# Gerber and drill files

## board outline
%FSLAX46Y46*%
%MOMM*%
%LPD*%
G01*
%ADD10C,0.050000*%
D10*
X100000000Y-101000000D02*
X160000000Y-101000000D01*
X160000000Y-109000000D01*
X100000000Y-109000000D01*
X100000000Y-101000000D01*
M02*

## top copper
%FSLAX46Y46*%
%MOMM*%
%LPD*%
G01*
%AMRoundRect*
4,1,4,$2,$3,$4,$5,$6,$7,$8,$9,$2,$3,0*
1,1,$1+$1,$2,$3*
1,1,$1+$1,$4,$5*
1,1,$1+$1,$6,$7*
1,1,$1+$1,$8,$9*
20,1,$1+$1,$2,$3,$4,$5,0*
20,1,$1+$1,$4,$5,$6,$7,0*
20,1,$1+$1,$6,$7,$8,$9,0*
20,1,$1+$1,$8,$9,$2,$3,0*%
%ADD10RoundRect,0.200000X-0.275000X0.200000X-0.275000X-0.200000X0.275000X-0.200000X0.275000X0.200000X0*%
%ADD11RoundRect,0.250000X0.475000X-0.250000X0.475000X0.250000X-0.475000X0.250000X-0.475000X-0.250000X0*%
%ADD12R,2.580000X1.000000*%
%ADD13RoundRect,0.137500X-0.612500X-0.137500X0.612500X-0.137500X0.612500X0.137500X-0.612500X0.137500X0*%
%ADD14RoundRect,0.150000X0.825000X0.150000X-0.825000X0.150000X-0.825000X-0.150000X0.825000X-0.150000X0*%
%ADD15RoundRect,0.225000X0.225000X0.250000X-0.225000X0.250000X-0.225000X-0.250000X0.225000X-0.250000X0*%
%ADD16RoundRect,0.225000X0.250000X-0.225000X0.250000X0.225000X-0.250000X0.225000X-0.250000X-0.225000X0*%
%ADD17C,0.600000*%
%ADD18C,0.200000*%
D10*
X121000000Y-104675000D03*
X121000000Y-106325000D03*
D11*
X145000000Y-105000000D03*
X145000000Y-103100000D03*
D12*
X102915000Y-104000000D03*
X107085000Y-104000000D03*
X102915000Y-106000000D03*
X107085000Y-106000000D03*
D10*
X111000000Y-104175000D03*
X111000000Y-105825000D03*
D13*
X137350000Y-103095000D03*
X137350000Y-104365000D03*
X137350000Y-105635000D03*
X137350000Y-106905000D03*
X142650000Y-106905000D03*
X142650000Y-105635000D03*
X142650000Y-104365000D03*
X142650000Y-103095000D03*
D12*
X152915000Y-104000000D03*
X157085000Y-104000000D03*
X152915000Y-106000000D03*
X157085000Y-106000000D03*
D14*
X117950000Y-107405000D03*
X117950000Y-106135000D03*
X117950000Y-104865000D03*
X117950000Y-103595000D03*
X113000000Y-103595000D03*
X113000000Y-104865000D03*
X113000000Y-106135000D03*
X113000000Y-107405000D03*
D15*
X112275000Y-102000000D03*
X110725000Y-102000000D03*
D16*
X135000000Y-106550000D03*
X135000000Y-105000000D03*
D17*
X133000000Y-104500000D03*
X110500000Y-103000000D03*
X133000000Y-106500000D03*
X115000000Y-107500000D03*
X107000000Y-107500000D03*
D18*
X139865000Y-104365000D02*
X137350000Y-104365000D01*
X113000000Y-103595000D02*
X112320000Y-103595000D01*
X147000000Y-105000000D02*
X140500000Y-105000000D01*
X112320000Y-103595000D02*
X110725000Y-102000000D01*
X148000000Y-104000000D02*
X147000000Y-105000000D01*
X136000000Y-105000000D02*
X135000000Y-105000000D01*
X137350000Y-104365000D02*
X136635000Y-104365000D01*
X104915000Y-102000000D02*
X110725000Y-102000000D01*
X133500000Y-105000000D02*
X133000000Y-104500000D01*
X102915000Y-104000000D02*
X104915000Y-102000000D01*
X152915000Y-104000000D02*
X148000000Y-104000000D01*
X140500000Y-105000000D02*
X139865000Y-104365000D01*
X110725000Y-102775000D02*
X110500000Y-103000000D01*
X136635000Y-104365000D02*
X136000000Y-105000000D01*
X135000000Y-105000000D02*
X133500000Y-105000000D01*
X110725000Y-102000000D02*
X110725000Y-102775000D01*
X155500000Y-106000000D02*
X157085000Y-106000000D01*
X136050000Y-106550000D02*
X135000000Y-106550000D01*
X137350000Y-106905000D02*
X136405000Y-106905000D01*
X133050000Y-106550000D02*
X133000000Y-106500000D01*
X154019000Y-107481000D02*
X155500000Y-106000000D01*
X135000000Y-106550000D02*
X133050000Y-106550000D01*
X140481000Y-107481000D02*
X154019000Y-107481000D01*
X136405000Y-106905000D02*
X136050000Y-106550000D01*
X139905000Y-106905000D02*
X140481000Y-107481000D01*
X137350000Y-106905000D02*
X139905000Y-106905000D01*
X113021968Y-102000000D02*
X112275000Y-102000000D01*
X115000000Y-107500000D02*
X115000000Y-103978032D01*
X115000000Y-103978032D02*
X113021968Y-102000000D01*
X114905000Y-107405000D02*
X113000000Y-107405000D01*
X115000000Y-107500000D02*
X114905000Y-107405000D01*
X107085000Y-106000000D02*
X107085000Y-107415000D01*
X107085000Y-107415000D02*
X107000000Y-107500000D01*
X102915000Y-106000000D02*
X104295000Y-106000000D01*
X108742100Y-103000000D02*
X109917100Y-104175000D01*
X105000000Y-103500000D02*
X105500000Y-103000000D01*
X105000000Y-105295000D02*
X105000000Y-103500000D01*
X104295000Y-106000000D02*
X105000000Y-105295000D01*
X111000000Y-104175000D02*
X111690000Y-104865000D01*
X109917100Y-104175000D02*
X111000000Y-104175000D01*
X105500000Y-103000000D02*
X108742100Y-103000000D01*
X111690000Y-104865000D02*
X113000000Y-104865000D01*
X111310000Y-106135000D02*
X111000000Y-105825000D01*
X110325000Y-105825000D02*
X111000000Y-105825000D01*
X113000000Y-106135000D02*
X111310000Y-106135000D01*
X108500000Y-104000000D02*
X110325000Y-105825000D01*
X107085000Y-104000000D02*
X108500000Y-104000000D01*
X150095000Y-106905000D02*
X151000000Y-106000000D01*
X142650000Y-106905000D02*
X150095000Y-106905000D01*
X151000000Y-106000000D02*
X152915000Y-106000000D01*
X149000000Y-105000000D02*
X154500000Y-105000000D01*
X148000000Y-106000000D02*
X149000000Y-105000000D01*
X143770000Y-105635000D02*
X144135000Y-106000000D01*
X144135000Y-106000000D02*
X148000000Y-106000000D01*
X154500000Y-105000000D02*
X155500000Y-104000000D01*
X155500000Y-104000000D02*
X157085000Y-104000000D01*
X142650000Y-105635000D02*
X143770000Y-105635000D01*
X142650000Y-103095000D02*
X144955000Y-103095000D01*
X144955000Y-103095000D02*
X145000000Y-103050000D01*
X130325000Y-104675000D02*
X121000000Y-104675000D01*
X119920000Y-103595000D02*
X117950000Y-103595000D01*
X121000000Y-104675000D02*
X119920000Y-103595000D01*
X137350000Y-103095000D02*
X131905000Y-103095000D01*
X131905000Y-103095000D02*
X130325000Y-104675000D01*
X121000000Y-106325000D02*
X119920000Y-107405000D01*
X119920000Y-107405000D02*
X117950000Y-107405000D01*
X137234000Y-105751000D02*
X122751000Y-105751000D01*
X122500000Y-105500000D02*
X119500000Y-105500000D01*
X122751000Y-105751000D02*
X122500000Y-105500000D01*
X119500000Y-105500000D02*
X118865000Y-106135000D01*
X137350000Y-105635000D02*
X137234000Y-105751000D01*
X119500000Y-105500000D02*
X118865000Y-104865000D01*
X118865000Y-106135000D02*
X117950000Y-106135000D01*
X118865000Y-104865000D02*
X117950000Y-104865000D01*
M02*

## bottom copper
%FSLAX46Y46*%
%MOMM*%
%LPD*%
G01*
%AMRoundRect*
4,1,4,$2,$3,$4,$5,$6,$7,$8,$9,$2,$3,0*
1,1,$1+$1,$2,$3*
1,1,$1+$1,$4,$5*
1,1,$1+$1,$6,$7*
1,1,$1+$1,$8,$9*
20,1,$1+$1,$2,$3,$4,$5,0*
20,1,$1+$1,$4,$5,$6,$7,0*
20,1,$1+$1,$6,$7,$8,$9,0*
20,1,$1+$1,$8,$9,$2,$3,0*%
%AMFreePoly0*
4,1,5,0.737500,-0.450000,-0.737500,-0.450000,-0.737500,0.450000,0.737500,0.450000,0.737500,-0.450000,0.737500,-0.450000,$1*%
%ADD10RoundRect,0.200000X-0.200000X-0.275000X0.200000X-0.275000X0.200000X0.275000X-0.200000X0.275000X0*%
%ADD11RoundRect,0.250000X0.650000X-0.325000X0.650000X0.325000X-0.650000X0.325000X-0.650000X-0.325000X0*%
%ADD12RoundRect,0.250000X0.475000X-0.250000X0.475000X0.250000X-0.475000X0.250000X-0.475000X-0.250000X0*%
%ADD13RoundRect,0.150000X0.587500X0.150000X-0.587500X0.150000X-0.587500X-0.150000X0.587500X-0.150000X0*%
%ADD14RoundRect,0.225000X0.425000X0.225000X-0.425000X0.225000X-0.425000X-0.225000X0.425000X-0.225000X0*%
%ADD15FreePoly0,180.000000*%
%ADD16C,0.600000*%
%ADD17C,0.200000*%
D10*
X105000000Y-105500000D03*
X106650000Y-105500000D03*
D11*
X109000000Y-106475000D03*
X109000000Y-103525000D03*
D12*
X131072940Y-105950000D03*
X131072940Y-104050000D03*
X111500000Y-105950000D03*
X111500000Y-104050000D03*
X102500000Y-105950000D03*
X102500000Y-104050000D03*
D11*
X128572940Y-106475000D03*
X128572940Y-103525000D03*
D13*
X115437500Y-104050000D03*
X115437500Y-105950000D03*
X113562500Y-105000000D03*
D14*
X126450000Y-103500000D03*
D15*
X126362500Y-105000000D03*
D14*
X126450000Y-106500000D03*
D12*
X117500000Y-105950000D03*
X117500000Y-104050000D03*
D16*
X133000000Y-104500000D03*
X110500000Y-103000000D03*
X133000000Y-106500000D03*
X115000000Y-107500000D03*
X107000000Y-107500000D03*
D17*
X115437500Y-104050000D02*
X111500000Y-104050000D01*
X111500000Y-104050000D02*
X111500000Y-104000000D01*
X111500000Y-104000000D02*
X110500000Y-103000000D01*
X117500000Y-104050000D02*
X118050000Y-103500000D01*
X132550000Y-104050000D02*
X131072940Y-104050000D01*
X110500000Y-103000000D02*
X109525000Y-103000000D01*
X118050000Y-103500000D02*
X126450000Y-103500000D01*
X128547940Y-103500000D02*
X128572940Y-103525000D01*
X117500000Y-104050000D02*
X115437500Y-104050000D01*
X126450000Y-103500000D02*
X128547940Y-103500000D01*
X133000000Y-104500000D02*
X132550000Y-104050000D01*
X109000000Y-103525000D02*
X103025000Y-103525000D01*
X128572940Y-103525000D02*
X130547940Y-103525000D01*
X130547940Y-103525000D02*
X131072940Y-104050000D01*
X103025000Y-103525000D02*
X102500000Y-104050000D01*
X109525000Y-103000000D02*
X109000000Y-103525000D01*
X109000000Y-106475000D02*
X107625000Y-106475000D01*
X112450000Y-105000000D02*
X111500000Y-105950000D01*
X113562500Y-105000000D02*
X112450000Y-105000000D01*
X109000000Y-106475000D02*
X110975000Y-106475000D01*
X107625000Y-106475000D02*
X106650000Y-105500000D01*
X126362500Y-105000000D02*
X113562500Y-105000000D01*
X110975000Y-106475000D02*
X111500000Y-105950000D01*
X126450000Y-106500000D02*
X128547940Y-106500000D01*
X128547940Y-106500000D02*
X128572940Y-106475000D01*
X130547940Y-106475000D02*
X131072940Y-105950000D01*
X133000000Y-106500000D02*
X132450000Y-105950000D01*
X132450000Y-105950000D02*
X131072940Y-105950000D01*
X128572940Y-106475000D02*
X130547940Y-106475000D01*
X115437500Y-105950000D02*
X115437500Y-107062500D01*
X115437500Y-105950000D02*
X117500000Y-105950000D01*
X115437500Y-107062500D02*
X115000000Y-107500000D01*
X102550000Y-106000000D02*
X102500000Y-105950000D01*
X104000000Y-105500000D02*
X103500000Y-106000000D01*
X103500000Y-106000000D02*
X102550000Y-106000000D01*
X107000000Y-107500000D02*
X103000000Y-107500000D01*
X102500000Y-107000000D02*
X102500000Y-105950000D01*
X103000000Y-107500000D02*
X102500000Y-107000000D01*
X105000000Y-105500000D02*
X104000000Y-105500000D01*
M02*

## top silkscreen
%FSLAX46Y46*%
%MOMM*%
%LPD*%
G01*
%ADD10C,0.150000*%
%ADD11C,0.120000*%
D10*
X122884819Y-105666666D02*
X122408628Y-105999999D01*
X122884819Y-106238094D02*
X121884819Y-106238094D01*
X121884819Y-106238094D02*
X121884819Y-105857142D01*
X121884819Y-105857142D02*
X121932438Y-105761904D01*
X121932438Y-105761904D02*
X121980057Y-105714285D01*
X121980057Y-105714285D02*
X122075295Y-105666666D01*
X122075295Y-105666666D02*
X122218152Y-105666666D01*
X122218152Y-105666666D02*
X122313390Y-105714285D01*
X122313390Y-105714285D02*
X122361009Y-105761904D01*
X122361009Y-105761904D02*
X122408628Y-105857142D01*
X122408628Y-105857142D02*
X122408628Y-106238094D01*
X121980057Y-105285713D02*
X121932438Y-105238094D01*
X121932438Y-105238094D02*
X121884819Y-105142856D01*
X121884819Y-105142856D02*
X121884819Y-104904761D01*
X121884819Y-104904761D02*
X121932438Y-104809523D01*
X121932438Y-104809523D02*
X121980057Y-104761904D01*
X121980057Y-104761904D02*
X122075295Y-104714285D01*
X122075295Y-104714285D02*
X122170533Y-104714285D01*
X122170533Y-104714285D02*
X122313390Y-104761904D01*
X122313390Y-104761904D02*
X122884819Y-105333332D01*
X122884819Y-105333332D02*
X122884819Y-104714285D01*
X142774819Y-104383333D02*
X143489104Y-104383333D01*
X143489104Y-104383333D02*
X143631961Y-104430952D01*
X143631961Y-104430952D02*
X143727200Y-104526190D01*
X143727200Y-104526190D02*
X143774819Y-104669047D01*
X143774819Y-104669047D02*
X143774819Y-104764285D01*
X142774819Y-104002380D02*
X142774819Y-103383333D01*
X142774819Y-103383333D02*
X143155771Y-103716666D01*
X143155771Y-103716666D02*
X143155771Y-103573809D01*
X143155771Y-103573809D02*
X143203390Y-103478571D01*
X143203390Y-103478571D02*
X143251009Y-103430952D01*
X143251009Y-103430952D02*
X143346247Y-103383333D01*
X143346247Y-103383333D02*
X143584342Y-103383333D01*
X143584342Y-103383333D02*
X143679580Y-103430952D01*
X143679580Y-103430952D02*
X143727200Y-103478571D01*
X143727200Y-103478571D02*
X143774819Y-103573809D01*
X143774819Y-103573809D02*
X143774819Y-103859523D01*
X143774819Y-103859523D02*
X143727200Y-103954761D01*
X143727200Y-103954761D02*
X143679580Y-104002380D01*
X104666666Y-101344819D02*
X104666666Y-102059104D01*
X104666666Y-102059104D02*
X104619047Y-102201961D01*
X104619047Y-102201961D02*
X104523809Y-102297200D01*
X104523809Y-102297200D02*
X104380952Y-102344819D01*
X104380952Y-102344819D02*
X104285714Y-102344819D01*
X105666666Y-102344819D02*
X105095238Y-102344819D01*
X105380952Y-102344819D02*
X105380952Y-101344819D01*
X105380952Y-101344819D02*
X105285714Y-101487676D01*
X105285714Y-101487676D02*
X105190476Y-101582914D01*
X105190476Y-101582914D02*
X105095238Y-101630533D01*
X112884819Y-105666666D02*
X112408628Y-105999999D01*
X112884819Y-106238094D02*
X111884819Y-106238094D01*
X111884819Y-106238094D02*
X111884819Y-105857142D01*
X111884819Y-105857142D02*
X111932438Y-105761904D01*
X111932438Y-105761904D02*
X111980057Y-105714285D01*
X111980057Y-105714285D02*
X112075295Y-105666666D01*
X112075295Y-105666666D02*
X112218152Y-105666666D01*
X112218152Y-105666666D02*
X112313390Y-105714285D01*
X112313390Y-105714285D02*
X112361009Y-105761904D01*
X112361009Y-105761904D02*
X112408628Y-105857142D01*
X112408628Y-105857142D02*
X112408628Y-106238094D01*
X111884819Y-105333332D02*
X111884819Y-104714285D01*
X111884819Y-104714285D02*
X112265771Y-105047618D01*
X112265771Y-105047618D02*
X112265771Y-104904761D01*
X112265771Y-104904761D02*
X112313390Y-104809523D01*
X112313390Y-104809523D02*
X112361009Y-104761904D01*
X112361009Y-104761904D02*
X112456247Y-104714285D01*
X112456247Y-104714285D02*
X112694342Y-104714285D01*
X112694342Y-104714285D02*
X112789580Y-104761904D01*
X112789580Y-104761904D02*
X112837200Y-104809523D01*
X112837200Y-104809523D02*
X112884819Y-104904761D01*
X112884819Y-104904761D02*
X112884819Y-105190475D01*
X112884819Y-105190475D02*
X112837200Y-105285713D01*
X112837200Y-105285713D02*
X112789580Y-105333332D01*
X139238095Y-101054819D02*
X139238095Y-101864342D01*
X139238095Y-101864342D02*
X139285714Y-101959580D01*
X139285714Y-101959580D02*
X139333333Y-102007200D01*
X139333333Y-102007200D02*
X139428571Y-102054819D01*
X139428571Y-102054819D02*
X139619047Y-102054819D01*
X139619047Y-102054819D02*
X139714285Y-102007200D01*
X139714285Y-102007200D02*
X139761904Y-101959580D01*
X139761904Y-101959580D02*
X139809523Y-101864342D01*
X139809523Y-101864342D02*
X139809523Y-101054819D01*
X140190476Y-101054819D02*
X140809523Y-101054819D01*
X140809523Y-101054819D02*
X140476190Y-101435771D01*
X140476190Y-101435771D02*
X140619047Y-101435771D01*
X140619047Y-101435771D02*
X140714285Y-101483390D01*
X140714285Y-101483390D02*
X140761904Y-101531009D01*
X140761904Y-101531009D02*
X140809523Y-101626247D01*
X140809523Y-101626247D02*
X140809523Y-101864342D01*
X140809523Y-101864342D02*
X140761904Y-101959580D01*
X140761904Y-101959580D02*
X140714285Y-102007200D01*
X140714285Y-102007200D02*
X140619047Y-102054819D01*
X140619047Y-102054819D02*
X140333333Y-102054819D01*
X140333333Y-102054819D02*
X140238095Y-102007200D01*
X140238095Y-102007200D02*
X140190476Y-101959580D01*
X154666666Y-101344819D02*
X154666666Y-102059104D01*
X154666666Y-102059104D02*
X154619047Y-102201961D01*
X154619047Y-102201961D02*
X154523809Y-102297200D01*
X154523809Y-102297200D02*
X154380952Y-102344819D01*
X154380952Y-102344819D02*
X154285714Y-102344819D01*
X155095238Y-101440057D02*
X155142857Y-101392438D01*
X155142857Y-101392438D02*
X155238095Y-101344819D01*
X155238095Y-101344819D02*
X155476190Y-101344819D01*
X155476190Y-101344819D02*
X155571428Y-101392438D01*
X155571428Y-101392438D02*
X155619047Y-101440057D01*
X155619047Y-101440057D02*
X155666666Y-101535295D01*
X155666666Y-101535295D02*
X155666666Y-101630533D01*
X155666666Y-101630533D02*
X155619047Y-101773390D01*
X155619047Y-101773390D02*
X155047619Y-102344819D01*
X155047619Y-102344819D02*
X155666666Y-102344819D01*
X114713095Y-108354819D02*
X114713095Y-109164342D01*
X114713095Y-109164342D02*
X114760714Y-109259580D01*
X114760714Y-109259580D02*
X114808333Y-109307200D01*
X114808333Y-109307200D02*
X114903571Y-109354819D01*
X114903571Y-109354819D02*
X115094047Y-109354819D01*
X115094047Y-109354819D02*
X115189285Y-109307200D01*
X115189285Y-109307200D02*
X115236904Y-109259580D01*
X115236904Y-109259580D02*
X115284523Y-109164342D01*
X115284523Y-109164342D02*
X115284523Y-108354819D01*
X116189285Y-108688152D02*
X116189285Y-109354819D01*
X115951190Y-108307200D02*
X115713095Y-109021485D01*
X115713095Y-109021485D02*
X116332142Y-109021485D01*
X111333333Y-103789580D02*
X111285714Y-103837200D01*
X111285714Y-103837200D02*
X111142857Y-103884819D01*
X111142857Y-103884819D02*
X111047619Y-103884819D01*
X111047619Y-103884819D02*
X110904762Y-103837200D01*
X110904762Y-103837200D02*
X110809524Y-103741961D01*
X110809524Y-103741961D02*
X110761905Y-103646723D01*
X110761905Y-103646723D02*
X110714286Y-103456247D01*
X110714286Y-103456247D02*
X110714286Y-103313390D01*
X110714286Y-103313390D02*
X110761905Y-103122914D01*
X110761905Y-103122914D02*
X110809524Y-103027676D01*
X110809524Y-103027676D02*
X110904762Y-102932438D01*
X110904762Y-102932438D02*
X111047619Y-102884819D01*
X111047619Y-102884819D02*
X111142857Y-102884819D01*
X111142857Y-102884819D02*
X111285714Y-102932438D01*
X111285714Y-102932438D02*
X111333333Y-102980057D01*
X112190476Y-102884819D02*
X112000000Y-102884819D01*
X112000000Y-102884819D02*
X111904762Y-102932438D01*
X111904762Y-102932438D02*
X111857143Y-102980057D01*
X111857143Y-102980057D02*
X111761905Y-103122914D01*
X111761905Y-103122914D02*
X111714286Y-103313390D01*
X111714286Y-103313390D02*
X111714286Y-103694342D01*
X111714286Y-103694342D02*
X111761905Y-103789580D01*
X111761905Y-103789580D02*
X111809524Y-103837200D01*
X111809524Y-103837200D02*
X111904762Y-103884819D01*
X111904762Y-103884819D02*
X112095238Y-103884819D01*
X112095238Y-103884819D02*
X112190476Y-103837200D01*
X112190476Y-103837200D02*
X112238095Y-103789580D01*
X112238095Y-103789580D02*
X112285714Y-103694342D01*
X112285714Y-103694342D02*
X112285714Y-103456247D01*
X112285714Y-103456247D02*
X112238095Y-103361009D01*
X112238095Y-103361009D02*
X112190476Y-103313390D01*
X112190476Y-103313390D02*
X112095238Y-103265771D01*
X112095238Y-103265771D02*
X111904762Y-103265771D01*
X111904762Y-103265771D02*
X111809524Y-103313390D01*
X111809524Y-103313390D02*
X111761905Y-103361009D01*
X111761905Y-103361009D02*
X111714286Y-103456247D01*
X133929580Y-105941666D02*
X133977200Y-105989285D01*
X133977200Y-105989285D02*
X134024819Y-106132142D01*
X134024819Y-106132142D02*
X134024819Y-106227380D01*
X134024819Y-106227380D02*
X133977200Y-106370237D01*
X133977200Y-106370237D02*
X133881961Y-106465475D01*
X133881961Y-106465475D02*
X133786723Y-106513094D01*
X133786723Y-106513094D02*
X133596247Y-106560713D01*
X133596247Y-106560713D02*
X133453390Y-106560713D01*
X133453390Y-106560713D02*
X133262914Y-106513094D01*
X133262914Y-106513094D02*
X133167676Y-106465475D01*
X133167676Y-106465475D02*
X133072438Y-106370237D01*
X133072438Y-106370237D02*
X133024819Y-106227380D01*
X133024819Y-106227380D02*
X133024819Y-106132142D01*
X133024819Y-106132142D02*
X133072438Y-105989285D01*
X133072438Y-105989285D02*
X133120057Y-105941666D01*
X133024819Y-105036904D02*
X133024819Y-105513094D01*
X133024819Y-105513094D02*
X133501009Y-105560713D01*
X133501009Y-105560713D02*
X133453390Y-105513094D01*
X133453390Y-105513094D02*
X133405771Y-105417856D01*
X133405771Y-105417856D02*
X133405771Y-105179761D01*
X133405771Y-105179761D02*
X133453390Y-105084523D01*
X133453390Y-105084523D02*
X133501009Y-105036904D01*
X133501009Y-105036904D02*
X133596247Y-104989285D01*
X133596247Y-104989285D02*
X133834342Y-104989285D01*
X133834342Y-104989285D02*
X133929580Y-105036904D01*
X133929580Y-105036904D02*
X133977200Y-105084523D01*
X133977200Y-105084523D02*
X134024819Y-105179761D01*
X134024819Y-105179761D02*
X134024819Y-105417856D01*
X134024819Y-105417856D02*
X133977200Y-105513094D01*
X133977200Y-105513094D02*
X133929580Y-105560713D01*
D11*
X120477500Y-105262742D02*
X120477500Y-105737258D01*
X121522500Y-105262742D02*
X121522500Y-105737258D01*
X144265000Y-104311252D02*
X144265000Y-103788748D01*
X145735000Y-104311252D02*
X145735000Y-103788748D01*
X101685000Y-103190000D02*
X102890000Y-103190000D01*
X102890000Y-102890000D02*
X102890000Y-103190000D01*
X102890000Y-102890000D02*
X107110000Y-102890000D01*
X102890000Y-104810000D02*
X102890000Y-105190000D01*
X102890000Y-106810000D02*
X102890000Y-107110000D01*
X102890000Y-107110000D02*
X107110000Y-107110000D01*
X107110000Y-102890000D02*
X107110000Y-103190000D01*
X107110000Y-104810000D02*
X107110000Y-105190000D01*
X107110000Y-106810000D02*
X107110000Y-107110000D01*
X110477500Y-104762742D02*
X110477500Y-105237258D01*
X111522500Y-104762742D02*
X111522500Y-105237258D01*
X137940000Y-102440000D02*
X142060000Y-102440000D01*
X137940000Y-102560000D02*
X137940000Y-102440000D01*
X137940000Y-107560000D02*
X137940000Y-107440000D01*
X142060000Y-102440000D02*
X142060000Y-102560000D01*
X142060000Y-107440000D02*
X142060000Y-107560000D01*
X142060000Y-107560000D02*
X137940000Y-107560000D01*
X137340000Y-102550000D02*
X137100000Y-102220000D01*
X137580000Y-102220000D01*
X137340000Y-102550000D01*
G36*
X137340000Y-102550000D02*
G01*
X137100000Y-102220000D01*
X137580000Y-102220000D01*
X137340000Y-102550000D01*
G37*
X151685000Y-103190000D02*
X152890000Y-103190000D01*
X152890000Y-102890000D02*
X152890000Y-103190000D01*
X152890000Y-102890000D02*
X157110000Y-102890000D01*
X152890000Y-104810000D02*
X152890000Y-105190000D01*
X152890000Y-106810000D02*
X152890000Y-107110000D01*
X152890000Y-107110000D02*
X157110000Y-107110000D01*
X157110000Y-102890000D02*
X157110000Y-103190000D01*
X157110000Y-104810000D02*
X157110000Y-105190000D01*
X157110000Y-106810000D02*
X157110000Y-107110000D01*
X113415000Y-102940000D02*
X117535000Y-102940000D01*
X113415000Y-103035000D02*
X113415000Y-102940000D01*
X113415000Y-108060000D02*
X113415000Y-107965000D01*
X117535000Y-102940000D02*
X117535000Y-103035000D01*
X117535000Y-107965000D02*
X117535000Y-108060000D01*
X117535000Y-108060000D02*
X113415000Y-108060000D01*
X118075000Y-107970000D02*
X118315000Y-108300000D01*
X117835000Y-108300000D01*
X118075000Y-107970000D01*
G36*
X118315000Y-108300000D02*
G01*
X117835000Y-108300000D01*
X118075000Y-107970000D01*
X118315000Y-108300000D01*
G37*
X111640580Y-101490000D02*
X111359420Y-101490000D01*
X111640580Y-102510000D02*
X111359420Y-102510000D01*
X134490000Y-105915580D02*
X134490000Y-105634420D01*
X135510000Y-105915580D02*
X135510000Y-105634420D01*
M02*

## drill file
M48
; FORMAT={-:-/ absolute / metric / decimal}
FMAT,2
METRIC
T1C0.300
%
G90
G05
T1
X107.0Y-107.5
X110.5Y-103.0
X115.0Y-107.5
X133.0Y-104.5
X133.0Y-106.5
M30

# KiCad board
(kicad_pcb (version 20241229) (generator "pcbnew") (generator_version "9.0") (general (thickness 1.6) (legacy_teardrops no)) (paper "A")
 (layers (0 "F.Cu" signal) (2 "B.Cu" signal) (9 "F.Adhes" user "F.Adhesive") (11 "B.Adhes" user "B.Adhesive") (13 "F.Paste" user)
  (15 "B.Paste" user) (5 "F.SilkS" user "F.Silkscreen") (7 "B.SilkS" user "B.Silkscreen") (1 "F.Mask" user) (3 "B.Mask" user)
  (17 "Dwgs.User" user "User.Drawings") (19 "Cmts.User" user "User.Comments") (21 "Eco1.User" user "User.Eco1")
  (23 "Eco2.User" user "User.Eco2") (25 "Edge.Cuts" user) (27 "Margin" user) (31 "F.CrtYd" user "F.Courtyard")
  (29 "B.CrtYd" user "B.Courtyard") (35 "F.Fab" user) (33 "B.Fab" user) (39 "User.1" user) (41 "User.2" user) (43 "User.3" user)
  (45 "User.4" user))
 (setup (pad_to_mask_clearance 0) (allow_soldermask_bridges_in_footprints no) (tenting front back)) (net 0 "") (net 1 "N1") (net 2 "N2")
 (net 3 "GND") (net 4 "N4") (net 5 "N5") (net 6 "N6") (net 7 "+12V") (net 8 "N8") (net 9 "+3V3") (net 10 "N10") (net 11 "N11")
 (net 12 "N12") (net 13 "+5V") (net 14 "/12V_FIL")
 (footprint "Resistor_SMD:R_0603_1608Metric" (layer "F.Cu") (at 121 105.5 -90)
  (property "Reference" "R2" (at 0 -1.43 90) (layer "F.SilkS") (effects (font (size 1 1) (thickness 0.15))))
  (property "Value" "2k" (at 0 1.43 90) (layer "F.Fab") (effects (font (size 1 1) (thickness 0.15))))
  (fp_line (start -0.237258 0.5225) (end 0.237258 0.5225) (stroke (width 0.12) (type solid)) (layer "F.SilkS"))
  (fp_line (start -0.237258 -0.5225) (end 0.237258 -0.5225) (stroke (width 0.12) (type solid)) (layer "F.SilkS"))
  (pad "1" smd roundrect (at -0.825 0 270) (size 0.8 0.95) (layers "F.Cu" "F.Mask" "F.Paste") (roundrect_rratio 0.25) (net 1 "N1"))
  (pad "2" smd roundrect (at 0.825 0 270) (size 0.8 0.95) (layers "F.Cu" "F.Mask" "F.Paste") (roundrect_rratio 0.25) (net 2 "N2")))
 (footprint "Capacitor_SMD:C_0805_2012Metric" (layer "F.Cu") (at 145 104.05 90)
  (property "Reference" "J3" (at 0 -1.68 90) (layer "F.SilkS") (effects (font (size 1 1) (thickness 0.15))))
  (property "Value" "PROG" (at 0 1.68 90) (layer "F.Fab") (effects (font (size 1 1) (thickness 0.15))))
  (fp_line (start -0.261252 -0.735) (end 0.261252 -0.735) (stroke (width 0.12) (type solid)) (layer "F.SilkS"))
  (fp_line (start -0.261252 0.735) (end 0.261252 0.735) (stroke (width 0.12) (type solid)) (layer "F.SilkS"))
  (pad "1" smd roundrect (at -0.95 0 90) (size 1 1.45) (layers "F.Cu" "F.Mask" "F.Paste") (roundrect_rratio 0.25) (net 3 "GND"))
  (pad "2" smd roundrect (at 0.95 0 90) (size 1 1.45) (layers "F.Cu" "F.Mask" "F.Paste") (roundrect_rratio 0.25) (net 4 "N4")))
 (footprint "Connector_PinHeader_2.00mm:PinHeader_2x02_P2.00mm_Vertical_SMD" (layer "F.Cu") (at 105 105)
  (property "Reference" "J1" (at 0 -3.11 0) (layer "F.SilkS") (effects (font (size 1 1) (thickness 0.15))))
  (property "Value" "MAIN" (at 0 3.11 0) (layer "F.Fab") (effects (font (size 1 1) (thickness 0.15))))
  (fp_line (start -3.315 -1.81) (end -2.11 -1.81) (stroke (width 0.12) (type solid)) (layer "F.SilkS"))
  (fp_line (start -2.11 -2.11) (end -2.11 -1.81) (stroke (width 0.12) (type solid)) (layer "F.SilkS"))
  (fp_line (start -2.11 -2.11) (end 2.11 -2.11) (stroke (width 0.12) (type solid)) (layer "F.SilkS"))
  (fp_line (start -2.11 -0.19) (end -2.11 0.19) (stroke (width 0.12) (type solid)) (layer "F.SilkS"))
  (fp_line (start -2.11 1.81) (end -2.11 2.11) (stroke (width 0.12) (type solid)) (layer "F.SilkS"))
  (fp_line (start -2.11 2.11) (end 2.11 2.11) (stroke (width 0.12) (type solid)) (layer "F.SilkS"))
  (fp_line (start 2.11 -2.11) (end 2.11 -1.81) (stroke (width 0.12) (type solid)) (layer "F.SilkS"))
  (fp_line (start 2.11 -0.19) (end 2.11 0.19) (stroke (width 0.12) (type solid)) (layer "F.SilkS"))
  (fp_line (start 2.11 1.81) (end 2.11 2.11) (stroke (width 0.12) (type solid)) (layer "F.SilkS"))
  (pad "1" smd rect (at -2.085 -1) (size 2.58 1) (layers "F.Cu" "F.Mask" "F.Paste") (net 3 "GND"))
  (pad "2" smd rect (at 2.085 -1) (size 2.58 1) (layers "F.Cu" "F.Mask" "F.Paste") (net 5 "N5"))
  (pad "3" smd rect (at -2.085 1) (size 2.58 1) (layers "F.Cu" "F.Mask" "F.Paste") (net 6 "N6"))
  (pad "4" smd rect (at 2.085 1) (size 2.58 1) (layers "F.Cu" "F.Mask" "F.Paste") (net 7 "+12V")))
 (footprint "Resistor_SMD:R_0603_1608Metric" (layer "F.Cu") (at 111 105 -90)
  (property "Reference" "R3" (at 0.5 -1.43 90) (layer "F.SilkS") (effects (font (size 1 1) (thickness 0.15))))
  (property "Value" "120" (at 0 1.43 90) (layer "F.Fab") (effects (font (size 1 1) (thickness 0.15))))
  (fp_line (start -0.237258 0.5225) (end 0.237258 0.5225) (stroke (width 0.12) (type solid)) (layer "F.SilkS"))
  (fp_line (start -0.237258 -0.5225) (end 0.237258 -0.5225) (stroke (width 0.12) (type solid)) (layer "F.SilkS"))
  (pad "1" smd roundrect (at -0.825 0 270) (size 0.8 0.95) (layers "F.Cu" "F.Mask" "F.Paste") (roundrect_rratio 0.25) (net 6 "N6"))
  (pad "2" smd roundrect (at 0.825 0 270) (size 0.8 0.95) (layers "F.Cu" "F.Mask" "F.Paste") (roundrect_rratio 0.25) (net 5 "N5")))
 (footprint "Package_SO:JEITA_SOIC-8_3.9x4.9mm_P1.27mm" (layer "F.Cu") (at 140 105)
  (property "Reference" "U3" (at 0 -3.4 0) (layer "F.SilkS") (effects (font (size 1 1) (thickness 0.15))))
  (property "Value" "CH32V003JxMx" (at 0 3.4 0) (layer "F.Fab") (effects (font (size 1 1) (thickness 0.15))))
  (fp_line (start -2.06 -2.56) (end 2.06 -2.56) (stroke (width 0.12) (type solid)) (layer "F.SilkS"))
  (fp_line (start -2.06 -2.44) (end -2.06 -2.56) (stroke (width 0.12) (type solid)) (layer "F.SilkS"))
  (fp_line (start -2.06 2.56) (end -2.06 2.44) (stroke (width 0.12) (type solid)) (layer "F.SilkS"))
  (fp_line (start 2.06 -2.56) (end 2.06 -2.44) (stroke (width 0.12) (type solid)) (layer "F.SilkS"))
  (fp_line (start 2.06 2.44) (end 2.06 2.56) (stroke (width 0.12) (type solid)) (layer "F.SilkS"))
  (fp_line (start 2.06 2.56) (end -2.06 2.56) (stroke (width 0.12) (type solid)) (layer "F.SilkS"))
  (fp_poly (pts (xy -2.66 -2.45) (xy -2.9 -2.78) (xy -2.42 -2.78)) (stroke (width 0.12) (type solid)) (fill yes) (layer "F.SilkS"))
  (pad "1" smd roundrect (at -2.65 -1.905) (size 1.5 0.55) (layers "F.Cu" "F.Mask" "F.Paste") (roundrect_rratio 0.25) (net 1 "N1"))
  (pad "2" smd roundrect (at -2.65 -0.635) (size 1.5 0.55) (layers "F.Cu" "F.Mask" "F.Paste") (roundrect_rratio 0.25) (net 3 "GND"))
  (pad "3" smd roundrect (at -2.65 0.635) (size 1.5 0.55) (layers "F.Cu" "F.Mask" "F.Paste") (roundrect_rratio 0.25) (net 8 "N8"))
  (pad "4" smd roundrect (at -2.65 1.905) (size 1.5 0.55) (layers "F.Cu" "F.Mask" "F.Paste") (roundrect_rratio 0.25) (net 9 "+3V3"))
  (pad "5" smd roundrect (at 2.65 1.905) (size 1.5 0.55) (layers "F.Cu" "F.Mask" "F.Paste") (roundrect_rratio 0.25) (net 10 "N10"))
  (pad "6" smd roundrect (at 2.65 0.635) (size 1.5 0.55) (layers "F.Cu" "F.Mask" "F.Paste") (roundrect_rratio 0.25) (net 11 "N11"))
  (pad "7" smd roundrect (at 2.65 -0.635) (size 1.5 0.55) (layers "F.Cu" "F.Mask" "F.Paste") (roundrect_rratio 0.25) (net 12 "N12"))
  (pad "8" smd roundrect (at 2.65 -1.905) (size 1.5 0.55) (layers "F.Cu" "F.Mask" "F.Paste") (roundrect_rratio 0.25) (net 4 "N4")))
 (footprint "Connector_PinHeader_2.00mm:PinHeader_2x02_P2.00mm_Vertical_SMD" (layer "F.Cu") (at 155 105)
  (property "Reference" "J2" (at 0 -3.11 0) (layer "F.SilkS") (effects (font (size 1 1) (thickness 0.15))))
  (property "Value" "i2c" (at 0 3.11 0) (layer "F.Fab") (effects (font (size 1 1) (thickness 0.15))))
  (fp_line (start -3.315 -1.81) (end -2.11 -1.81) (stroke (width 0.12) (type solid)) (layer "F.SilkS"))
  (fp_line (start -2.11 -2.11) (end -2.11 -1.81) (stroke (width 0.12) (type solid)) (layer "F.SilkS"))
  (fp_line (start -2.11 -2.11) (end 2.11 -2.11) (stroke (width 0.12) (type solid)) (layer "F.SilkS"))
  (fp_line (start -2.11 -0.19) (end -2.11 0.19) (stroke (width 0.12) (type solid)) (layer "F.SilkS"))
  (fp_line (start -2.11 1.81) (end -2.11 2.11) (stroke (width 0.12) (type solid)) (layer "F.SilkS"))
  (fp_line (start -2.11 2.11) (end 2.11 2.11) (stroke (width 0.12) (type solid)) (layer "F.SilkS"))
  (fp_line (start 2.11 -2.11) (end 2.11 -1.81) (stroke (width 0.12) (type solid)) (layer "F.SilkS"))
  (fp_line (start 2.11 -0.19) (end 2.11 0.19) (stroke (width 0.12) (type solid)) (layer "F.SilkS"))
  (fp_line (start 2.11 1.81) (end 2.11 2.11) (stroke (width 0.12) (type solid)) (layer "F.SilkS"))
  (pad "1" smd rect (at -2.085 -1) (size 2.58 1) (layers "F.Cu" "F.Mask" "F.Paste") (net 3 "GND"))
  (pad "2" smd rect (at 2.085 -1) (size 2.58 1) (layers "F.Cu" "F.Mask" "F.Paste") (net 11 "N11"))
  (pad "3" smd rect (at -2.085 1) (size 2.58 1) (layers "F.Cu" "F.Mask" "F.Paste") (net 10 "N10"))
  (pad "4" smd rect (at 2.085 1) (size 2.58 1) (layers "F.Cu" "F.Mask" "F.Paste") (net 9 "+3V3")))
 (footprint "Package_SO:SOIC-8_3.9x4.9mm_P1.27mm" (layer "F.Cu") (at 115.475 105.5 180)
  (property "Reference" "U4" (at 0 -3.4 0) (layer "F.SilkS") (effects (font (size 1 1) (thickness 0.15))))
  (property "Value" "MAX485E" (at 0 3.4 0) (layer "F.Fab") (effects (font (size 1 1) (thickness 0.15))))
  (fp_line (start 2.06 2.56) (end -2.06 2.56) (stroke (width 0.12) (type solid)) (layer "F.SilkS"))
  (fp_line (start 2.06 2.465) (end 2.06 2.56) (stroke (width 0.12) (type solid)) (layer "F.SilkS"))
  (fp_line (start 2.06 -2.56) (end 2.06 -2.465) (stroke (width 0.12) (type solid)) (layer "F.SilkS"))
  (fp_line (start -2.06 2.56) (end -2.06 2.465) (stroke (width 0.12) (type solid)) (layer "F.SilkS"))
  (fp_line (start -2.06 -2.465) (end -2.06 -2.56) (stroke (width 0.12) (type solid)) (layer "F.SilkS"))
  (fp_line (start -2.06 -2.56) (end 2.06 -2.56) (stroke (width 0.12) (type solid)) (layer "F.SilkS"))
  (fp_poly (pts (xy -2.6 -2.47) (xy -2.84 -2.8) (xy -2.36 -2.8)) (stroke (width 0.12) (type solid)) (fill yes) (layer "F.SilkS"))
  (pad "1" smd roundrect (at -2.475 -1.905 180) (size 1.95 0.6) (layers "F.Cu" "F.Mask" "F.Paste") (roundrect_rratio 0.25) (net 2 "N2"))
  (pad "2" smd roundrect (at -2.475 -0.635 180) (size 1.95 0.6) (layers "F.Cu" "F.Mask" "F.Paste") (roundrect_rratio 0.25) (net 8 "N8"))
  (pad "3" smd roundrect (at -2.475 0.635 180) (size 1.95 0.6) (layers "F.Cu" "F.Mask" "F.Paste") (roundrect_rratio 0.25) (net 8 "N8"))
  (pad "4" smd roundrect (at -2.475 1.905 180) (size 1.95 0.6) (layers "F.Cu" "F.Mask" "F.Paste") (roundrect_rratio 0.25) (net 1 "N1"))
  (pad "5" smd roundrect (at 2.475 1.905 180) (size 1.95 0.6) (layers "F.Cu" "F.Mask" "F.Paste") (roundrect_rratio 0.25) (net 3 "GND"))
  (pad "6" smd roundrect (at 2.475 0.635 180) (size 1.95 0.6) (layers "F.Cu" "F.Mask" "F.Paste") (roundrect_rratio 0.25) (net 6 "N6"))
  (pad "7" smd roundrect (at 2.475 -0.635 180) (size 1.95 0.6) (layers "F.Cu" "F.Mask" "F.Paste") (roundrect_rratio 0.25) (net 5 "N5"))
  (pad "8" smd roundrect (at 2.475 -1.905 180) (size 1.95 0.6) (layers "F.Cu" "F.Mask" "F.Paste") (roundrect_rratio 0.25) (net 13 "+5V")))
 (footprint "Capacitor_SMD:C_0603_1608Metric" (layer "F.Cu") (at 111.5 102 180)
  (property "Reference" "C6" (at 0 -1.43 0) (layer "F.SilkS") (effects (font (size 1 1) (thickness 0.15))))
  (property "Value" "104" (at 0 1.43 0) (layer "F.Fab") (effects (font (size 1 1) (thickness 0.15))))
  (fp_line (start -0.14058 0.51) (end 0.14058 0.51) (stroke (width 0.12) (type solid)) (layer "F.SilkS"))
  (fp_line (start -0.14058 -0.51) (end 0.14058 -0.51) (stroke (width 0.12) (type solid)) (layer "F.SilkS"))
  (pad "1" smd roundrect (at -0.775 0 180) (size 0.9 0.95) (layers "F.Cu" "F.Mask" "F.Paste") (roundrect_rratio 0.25) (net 13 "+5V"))
  (pad "2" smd roundrect (at 0.775 0 180) (size 0.9 0.95) (layers "F.Cu" "F.Mask" "F.Paste") (roundrect_rratio 0.25) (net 3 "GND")))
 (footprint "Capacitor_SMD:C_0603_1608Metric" (layer "F.Cu") (at 135 105.775 90)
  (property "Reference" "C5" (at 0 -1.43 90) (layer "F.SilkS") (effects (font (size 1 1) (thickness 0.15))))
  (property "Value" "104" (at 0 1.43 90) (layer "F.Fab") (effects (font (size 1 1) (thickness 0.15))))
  (fp_line (start -0.14058 -0.51) (end 0.14058 -0.51) (stroke (width 0.12) (type solid)) (layer "F.SilkS"))
  (fp_line (start -0.14058 0.51) (end 0.14058 0.51) (stroke (width 0.12) (type solid)) (layer "F.SilkS"))
  (pad "1" smd roundrect (at -0.775 0 90) (size 0.9 0.95) (layers "F.Cu" "F.Mask" "F.Paste") (roundrect_rratio 0.25) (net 9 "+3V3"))
  (pad "2" smd roundrect (at 0.775 0 90) (size 0.9 0.95) (layers "F.Cu" "F.Mask" "F.Paste") (roundrect_rratio 0.25) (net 3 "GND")))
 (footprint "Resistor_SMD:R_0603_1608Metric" (layer "B.Cu") (at 105.825 105.5)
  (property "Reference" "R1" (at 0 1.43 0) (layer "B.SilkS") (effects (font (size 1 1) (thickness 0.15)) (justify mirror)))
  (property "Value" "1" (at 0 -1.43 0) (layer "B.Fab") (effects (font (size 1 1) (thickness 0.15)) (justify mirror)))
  (pad "1" smd roundrect (at -0.825 0) (size 0.8 0.95) (layers "B.Cu" "B.Mask" "B.Paste") (roundrect_rratio 0.25) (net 7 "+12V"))
  (pad "2" smd roundrect (at 0.825 0) (size 0.8 0.95) (layers "B.Cu" "B.Mask" "B.Paste") (roundrect_rratio 0.25) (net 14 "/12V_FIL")))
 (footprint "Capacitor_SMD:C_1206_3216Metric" (layer "B.Cu") (at 109 105 90)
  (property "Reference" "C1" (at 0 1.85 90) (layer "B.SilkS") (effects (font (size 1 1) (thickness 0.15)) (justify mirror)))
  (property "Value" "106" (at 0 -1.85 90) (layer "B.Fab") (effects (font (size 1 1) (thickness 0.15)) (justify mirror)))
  (pad "1" smd roundrect (at -1.475 0 90) (size 1.15 1.8) (layers "B.Cu" "B.Mask" "B.Paste") (roundrect_rratio 0.217391) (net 14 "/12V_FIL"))
  (pad "2" smd roundrect (at 1.475 0 90) (size 1.15 1.8) (layers "B.Cu" "B.Mask" "B.Paste") (roundrect_rratio 0.217391) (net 3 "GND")))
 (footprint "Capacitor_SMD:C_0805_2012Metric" (layer "B.Cu") (at 131.07294 105 90)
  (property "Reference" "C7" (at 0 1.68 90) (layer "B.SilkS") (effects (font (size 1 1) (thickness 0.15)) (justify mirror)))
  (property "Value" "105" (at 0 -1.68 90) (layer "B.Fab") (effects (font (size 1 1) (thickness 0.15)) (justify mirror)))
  (pad "1" smd roundrect (at -0.95 0 90) (size 1 1.45) (layers "B.Cu" "B.Mask" "B.Paste") (roundrect_rratio 0.25) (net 9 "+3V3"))
  (pad "2" smd roundrect (at 0.95 0 90) (size 1 1.45) (layers "B.Cu" "B.Mask" "B.Paste") (roundrect_rratio 0.25) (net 3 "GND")))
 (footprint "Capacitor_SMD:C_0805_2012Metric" (layer "B.Cu") (at 111.5 105 90)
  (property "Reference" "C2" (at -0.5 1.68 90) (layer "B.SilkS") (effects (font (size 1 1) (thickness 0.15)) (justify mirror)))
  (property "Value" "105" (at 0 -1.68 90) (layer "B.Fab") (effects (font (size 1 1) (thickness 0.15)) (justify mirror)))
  (pad "1" smd roundrect (at -0.95 0 90) (size 1 1.45) (layers "B.Cu" "B.Mask" "B.Paste") (roundrect_rratio 0.25) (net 14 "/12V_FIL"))
  (pad "2" smd roundrect (at 0.95 0 90) (size 1 1.45) (layers "B.Cu" "B.Mask" "B.Paste") (roundrect_rratio 0.25) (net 3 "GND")))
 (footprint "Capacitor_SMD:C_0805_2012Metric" (layer "B.Cu") (at 102.5 105 90)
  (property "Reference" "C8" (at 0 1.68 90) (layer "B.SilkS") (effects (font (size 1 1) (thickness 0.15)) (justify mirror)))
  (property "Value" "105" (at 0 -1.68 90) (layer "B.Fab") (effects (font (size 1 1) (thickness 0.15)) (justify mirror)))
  (pad "1" smd roundrect (at -0.95 0 90) (size 1 1.45) (layers "B.Cu" "B.Mask" "B.Paste") (roundrect_rratio 0.25) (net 7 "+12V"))
  (pad "2" smd roundrect (at 0.95 0 90) (size 1 1.45) (layers "B.Cu" "B.Mask" "B.Paste") (roundrect_rratio 0.25) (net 3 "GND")))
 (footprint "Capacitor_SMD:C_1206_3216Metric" (layer "B.Cu") (at 128.57294 105 90)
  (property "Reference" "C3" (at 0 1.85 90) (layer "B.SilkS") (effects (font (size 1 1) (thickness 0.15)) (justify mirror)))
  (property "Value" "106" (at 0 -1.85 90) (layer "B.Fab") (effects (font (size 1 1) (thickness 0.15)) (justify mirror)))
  (pad "1" smd roundrect (at -1.475 0 90) (size 1.15 1.8) (layers "B.Cu" "B.Mask" "B.Paste") (roundrect_rratio 0.217391) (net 9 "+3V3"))
  (pad "2" smd roundrect (at 1.475 0 90) (size 1.15 1.8) (layers "B.Cu" "B.Mask" "B.Paste") (roundrect_rratio 0.217391) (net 3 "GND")))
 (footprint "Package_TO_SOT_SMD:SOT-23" (layer "B.Cu") (at 114.5 105 180)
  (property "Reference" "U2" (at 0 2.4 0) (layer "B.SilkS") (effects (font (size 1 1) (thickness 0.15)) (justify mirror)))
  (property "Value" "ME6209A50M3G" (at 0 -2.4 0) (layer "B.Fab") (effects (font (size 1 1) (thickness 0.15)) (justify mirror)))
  (pad "1" smd roundrect (at -0.9375 0.95 180) (size 1.475 0.6) (layers "B.Cu" "B.Mask" "B.Paste") (roundrect_rratio 0.25) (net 3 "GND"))
  (pad "2" smd roundrect (at -0.9375 -0.95 180) (size 1.475 0.6) (layers "B.Cu" "B.Mask" "B.Paste") (roundrect_rratio 0.25) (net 13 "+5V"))
  (pad "3" smd roundrect (at 0.9375 0 180) (size 1.475 0.6) (layers "B.Cu" "B.Mask" "B.Paste") (roundrect_rratio 0.25) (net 14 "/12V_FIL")))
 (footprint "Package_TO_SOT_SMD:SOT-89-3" (layer "B.Cu") (at 124.5 105 180)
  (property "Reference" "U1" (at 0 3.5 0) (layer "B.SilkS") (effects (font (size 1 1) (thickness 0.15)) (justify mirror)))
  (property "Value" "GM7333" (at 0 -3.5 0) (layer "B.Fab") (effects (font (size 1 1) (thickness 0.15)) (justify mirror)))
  (pad "1" smd roundrect (at -1.95 1.5 180) (size 1.3 0.9) (layers "B.Cu" "B.Mask" "B.Paste") (roundrect_rratio 0.25) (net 3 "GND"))
  (pad "2" smd custom (at -1.8625 0 180) (size 1.475 0.9) (layers "B.Cu" "B.Mask" "B.Paste") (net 14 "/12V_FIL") (zone_connect 2)
   (thermal_bridge_angle 45) (options (clearance outline) (anchor rect)) (primitives))
  (pad "3" smd roundrect (at -1.95 -1.5 180) (size 1.3 0.9) (layers "B.Cu" "B.Mask" "B.Paste") (roundrect_rratio 0.25) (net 9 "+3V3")))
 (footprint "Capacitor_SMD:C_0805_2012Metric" (layer "B.Cu") (at 117.5 105 90)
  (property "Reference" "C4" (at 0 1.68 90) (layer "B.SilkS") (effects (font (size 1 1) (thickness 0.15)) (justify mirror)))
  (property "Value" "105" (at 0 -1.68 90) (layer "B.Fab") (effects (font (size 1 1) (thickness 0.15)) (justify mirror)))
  (pad "1" smd roundrect (at -0.95 0 90) (size 1 1.45) (layers "B.Cu" "B.Mask" "B.Paste") (roundrect_rratio 0.25) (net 13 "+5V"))
  (pad "2" smd roundrect (at 0.95 0 90) (size 1 1.45) (layers "B.Cu" "B.Mask" "B.Paste") (roundrect_rratio 0.25) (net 3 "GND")))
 (gr_rect (start 100 101) (end 160 109) (stroke (width 0.05) (type solid)) (fill no) (layer "Edge.Cuts"))
 (segment (start 139.865 104.365) (end 137.35 104.365) (width 0.2) (layer "F.Cu") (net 3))
 (segment (start 113 103.595) (end 112.32 103.595) (width 0.2) (layer "F.Cu") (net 3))
 (segment (start 147 105) (end 140.5 105) (width 0.2) (layer "F.Cu") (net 3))
 (segment (start 112.32 103.595) (end 110.725 102) (width 0.2) (layer "F.Cu") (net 3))
 (segment (start 148 104) (end 147 105) (width 0.2) (layer "F.Cu") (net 3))
 (segment (start 136 105) (end 135 105) (width 0.2) (layer "F.Cu") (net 3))
 (segment (start 137.35 104.365) (end 136.635 104.365) (width 0.2) (layer "F.Cu") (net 3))
 (segment (start 104.915 102) (end 110.725 102) (width 0.2) (layer "F.Cu") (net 3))
 (segment (start 133.5 105) (end 133 104.5) (width 0.2) (layer "F.Cu") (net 3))
 (segment (start 102.915 104) (end 104.915 102) (width 0.2) (layer "F.Cu") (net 3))
 (segment (start 152.915 104) (end 148 104) (width 0.2) (layer "F.Cu") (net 3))
 (segment (start 140.5 105) (end 139.865 104.365) (width 0.2) (layer "F.Cu") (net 3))
 (segment (start 110.725 102.775) (end 110.5 103) (width 0.2) (layer "F.Cu") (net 3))
 (segment (start 136.635 104.365) (end 136 105) (width 0.2) (layer "F.Cu") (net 3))
 (segment (start 135 105) (end 133.5 105) (width 0.2) (layer "F.Cu") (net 3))
 (segment (start 110.725 102) (end 110.725 102.775) (width 0.2) (layer "F.Cu") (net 3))
 (via (at 133 104.5) (size 0.6) (drill 0.3) (layers "F.Cu" "B.Cu") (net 3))
 (via (at 110.5 103) (size 0.6) (drill 0.3) (layers "F.Cu" "B.Cu") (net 3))
 (segment (start 115.4375 104.05) (end 111.5 104.05) (width 0.2) (layer "B.Cu") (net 3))
 (segment (start 111.5 104.05) (end 111.5 104) (width 0.2) (layer "B.Cu") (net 3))
 (segment (start 111.5 104) (end 110.5 103) (width 0.2) (layer "B.Cu") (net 3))
 (segment (start 117.5 104.05) (end 118.05 103.5) (width 0.2) (layer "B.Cu") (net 3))
 (segment (start 132.55 104.05) (end 131.07294 104.05) (width 0.2) (layer "B.Cu") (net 3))
 (segment (start 110.5 103) (end 109.525 103) (width 0.2) (layer "B.Cu") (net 3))
 (segment (start 118.05 103.5) (end 126.45 103.5) (width 0.2) (layer "B.Cu") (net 3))
 (segment (start 128.54794 103.5) (end 128.57294 103.525) (width 0.2) (layer "B.Cu") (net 3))
 (segment (start 117.5 104.05) (end 115.4375 104.05) (width 0.2) (layer "B.Cu") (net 3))
 (segment (start 126.45 103.5) (end 128.54794 103.5) (width 0.2) (layer "B.Cu") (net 3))
 (segment (start 133 104.5) (end 132.55 104.05) (width 0.2) (layer "B.Cu") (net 3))
 (segment (start 109 103.525) (end 103.025 103.525) (width 0.2) (layer "B.Cu") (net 3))
 (segment (start 128.57294 103.525) (end 130.54794 103.525) (width 0.2) (layer "B.Cu") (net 3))
 (segment (start 130.54794 103.525) (end 131.07294 104.05) (width 0.2) (layer "B.Cu") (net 3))
 (segment (start 103.025 103.525) (end 102.5 104.05) (width 0.2) (layer "B.Cu") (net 3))
 (segment (start 109.525 103) (end 109 103.525) (width 0.2) (layer "B.Cu") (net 3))
 (segment (start 109 106.475) (end 107.625 106.475) (width 0.2) (layer "B.Cu") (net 14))
 (segment (start 112.45 105) (end 111.5 105.95) (width 0.2) (layer "B.Cu") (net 14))
 (segment (start 113.5625 105) (end 112.45 105) (width 0.2) (layer "B.Cu") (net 14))
 (segment (start 109 106.475) (end 110.975 106.475) (width 0.2) (layer "B.Cu") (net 14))
 (segment (start 107.625 106.475) (end 106.65 105.5) (width 0.2) (layer "B.Cu") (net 14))
 (segment (start 126.3625 105) (end 113.5625 105) (width 0.2) (layer "B.Cu") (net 14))
 (segment (start 110.975 106.475) (end 111.5 105.95) (width 0.2) (layer "B.Cu") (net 14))
 (segment (start 155.5 106) (end 157.085 106) (width 0.2) (layer "F.Cu") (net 9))
 (segment (start 136.05 106.55) (end 135 106.55) (width 0.2) (layer "F.Cu") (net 9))
 (segment (start 137.35 106.905) (end 136.405 106.905) (width 0.2) (layer "F.Cu") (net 9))
 (segment (start 133.05 106.55) (end 133 106.5) (width 0.2) (layer "F.Cu") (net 9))
 (segment (start 154.019 107.481) (end 155.5 106) (width 0.2) (layer "F.Cu") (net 9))
 (segment (start 135 106.55) (end 133.05 106.55) (width 0.2) (layer "F.Cu") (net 9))
 (segment (start 140.481 107.481) (end 154.019 107.481) (width 0.2) (layer "F.Cu") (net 9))
 (segment (start 136.405 106.905) (end 136.05 106.55) (width 0.2) (layer "F.Cu") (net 9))
 (segment (start 139.905 106.905) (end 140.481 107.481) (width 0.2) (layer "F.Cu") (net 9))
 (segment (start 137.35 106.905) (end 139.905 106.905) (width 0.2) (layer "F.Cu") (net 9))
 (via (at 133 106.5) (size 0.6) (drill 0.3) (layers "F.Cu" "B.Cu") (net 9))
 (segment (start 126.45 106.5) (end 128.54794 106.5) (width 0.2) (layer "B.Cu") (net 9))
 (segment (start 128.54794 106.5) (end 128.57294 106.475) (width 0.2) (layer "B.Cu") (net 9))
 (segment (start 130.54794 106.475) (end 131.07294 105.95) (width 0.2) (layer "B.Cu") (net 9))
 (segment (start 133 106.5) (end 132.45 105.95) (width 0.2) (layer "B.Cu") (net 9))
 (segment (start 132.45 105.95) (end 131.07294 105.95) (width 0.2) (layer "B.Cu") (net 9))
 (segment (start 128.57294 106.475) (end 130.54794 106.475) (width 0.2) (layer "B.Cu") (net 9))
 (segment (start 113.021968 102) (end 112.275 102) (width 0.2) (layer "F.Cu") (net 13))
 (segment (start 115 107.5) (end 115 103.978032) (width 0.2) (layer "F.Cu") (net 13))
 (segment (start 115 103.978032) (end 113.021968 102) (width 0.2) (layer "F.Cu") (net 13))
 (segment (start 114.905 107.405) (end 113 107.405) (width 0.2) (layer "F.Cu") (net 13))
 (segment (start 115 107.5) (end 114.905 107.405) (width 0.2) (layer "F.Cu") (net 13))
 (via (at 115 107.5) (size 0.6) (drill 0.3) (layers "F.Cu" "B.Cu") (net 13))
 (segment (start 115.4375 105.95) (end 115.4375 107.0625) (width 0.2) (layer "B.Cu") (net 13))
 (segment (start 115.4375 105.95) (end 117.5 105.95) (width 0.2) (layer "B.Cu") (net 13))
 (segment (start 115.4375 107.0625) (end 115 107.5) (width 0.2) (layer "B.Cu") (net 13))
 (segment (start 107.085 106) (end 107.085 107.415) (width 0.2) (layer "F.Cu") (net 7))
 (segment (start 107.085 107.415) (end 107 107.5) (width 0.2) (layer "F.Cu") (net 7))
 (via (at 107 107.5) (size 0.6) (drill 0.3) (layers "F.Cu" "B.Cu") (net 7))
 (segment (start 102.55 106) (end 102.5 105.95) (width 0.2) (layer "B.Cu") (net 7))
 (segment (start 104 105.5) (end 103.5 106) (width 0.2) (layer "B.Cu") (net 7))
 (segment (start 103.5 106) (end 102.55 106) (width 0.2) (layer "B.Cu") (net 7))
 (segment (start 107 107.5) (end 103 107.5) (width 0.2) (layer "B.Cu") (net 7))
 (segment (start 102.5 107) (end 102.5 105.95) (width 0.2) (layer "B.Cu") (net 7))
 (segment (start 103 107.5) (end 102.5 107) (width 0.2) (layer "B.Cu") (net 7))
 (segment (start 105 105.5) (end 104 105.5) (width 0.2) (layer "B.Cu") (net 7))
 (segment (start 102.915 106) (end 104.295 106) (width 0.2) (layer "F.Cu") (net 6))
 (segment (start 108.7421 103) (end 109.9171 104.175) (width 0.2) (layer "F.Cu") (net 6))
 (segment (start 105 103.5) (end 105.5 103) (width 0.2) (layer "F.Cu") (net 6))
 (segment (start 105 105.295) (end 105 103.5) (width 0.2) (layer "F.Cu") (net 6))
 (segment (start 104.295 106) (end 105 105.295) (width 0.2) (layer "F.Cu") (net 6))
 (segment (start 111 104.175) (end 111.69 104.865) (width 0.2) (layer "F.Cu") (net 6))
 (segment (start 109.9171 104.175) (end 111 104.175) (width 0.2) (layer "F.Cu") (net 6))
 (segment (start 105.5 103) (end 108.7421 103) (width 0.2) (layer "F.Cu") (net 6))
 (segment (start 111.69 104.865) (end 113 104.865) (width 0.2) (layer "F.Cu") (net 6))
 (segment (start 111.31 106.135) (end 111 105.825) (width 0.2) (layer "F.Cu") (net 5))
 (segment (start 110.325 105.825) (end 111 105.825) (width 0.2) (layer "F.Cu") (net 5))
 (segment (start 113 106.135) (end 111.31 106.135) (width 0.2) (layer "F.Cu") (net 5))
 (segment (start 108.5 104) (end 110.325 105.825) (width 0.2) (layer "F.Cu") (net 5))
 (segment (start 107.085 104) (end 108.5 104) (width 0.2) (layer "F.Cu") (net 5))
 (segment (start 150.095 106.905) (end 151 106) (width 0.2) (layer "F.Cu") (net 10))
 (segment (start 142.65 106.905) (end 150.095 106.905) (width 0.2) (layer "F.Cu") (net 10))
 (segment (start 151 106) (end 152.915 106) (width 0.2) (layer "F.Cu") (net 10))
 (segment (start 149 105) (end 154.5 105) (width 0.2) (layer "F.Cu") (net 11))
 (segment (start 148 106) (end 149 105) (width 0.2) (layer "F.Cu") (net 11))
 (segment (start 143.77 105.635) (end 144.135 106) (width 0.2) (layer "F.Cu") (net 11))
 (segment (start 144.135 106) (end 148 106) (width 0.2) (layer "F.Cu") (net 11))
 (segment (start 154.5 105) (end 155.5 104) (width 0.2) (layer "F.Cu") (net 11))
 (segment (start 155.5 104) (end 157.085 104) (width 0.2) (layer "F.Cu") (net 11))
 (segment (start 142.65 105.635) (end 143.77 105.635) (width 0.2) (layer "F.Cu") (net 11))
 (segment (start 142.65 103.095) (end 144.955 103.095) (width 0.2) (layer "F.Cu") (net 4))
 (segment (start 144.955 103.095) (end 145 103.05) (width 0.2) (layer "F.Cu") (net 4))
 (segment (start 130.325 104.675) (end 121 104.675) (width 0.2) (layer "F.Cu") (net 1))
 (segment (start 119.92 103.595) (end 117.95 103.595) (width 0.2) (layer "F.Cu") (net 1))
 (segment (start 121 104.675) (end 119.92 103.595) (width 0.2) (layer "F.Cu") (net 1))
 (segment (start 137.35 103.095) (end 131.905 103.095) (width 0.2) (layer "F.Cu") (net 1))
 (segment (start 131.905 103.095) (end 130.325 104.675) (width 0.2) (layer "F.Cu") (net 1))
 (segment (start 121 106.325) (end 119.92 107.405) (width 0.2) (layer "F.Cu") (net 2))
 (segment (start 119.92 107.405) (end 117.95 107.405) (width 0.2) (layer "F.Cu") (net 2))
 (segment (start 137.234 105.751) (end 122.751 105.751) (width 0.2) (layer "F.Cu") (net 8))
 (segment (start 122.5 105.5) (end 119.5 105.5) (width 0.2) (layer "F.Cu") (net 8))
 (segment (start 122.751 105.751) (end 122.5 105.5) (width 0.2) (layer "F.Cu") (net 8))
 (segment (start 119.5 105.5) (end 118.865 106.135) (width 0.2) (layer "F.Cu") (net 8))
 (segment (start 137.35 105.635) (end 137.234 105.751) (width 0.2) (layer "F.Cu") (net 8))
 (segment (start 119.5 105.5) (end 118.865 104.865) (width 0.2) (layer "F.Cu") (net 8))
 (segment (start 118.865 106.135) (end 117.95 106.135) (width 0.2) (layer "F.Cu") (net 8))
 (segment (start 118.865 104.865) (end 117.95 104.865) (width 0.2) (layer "F.Cu") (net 8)))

